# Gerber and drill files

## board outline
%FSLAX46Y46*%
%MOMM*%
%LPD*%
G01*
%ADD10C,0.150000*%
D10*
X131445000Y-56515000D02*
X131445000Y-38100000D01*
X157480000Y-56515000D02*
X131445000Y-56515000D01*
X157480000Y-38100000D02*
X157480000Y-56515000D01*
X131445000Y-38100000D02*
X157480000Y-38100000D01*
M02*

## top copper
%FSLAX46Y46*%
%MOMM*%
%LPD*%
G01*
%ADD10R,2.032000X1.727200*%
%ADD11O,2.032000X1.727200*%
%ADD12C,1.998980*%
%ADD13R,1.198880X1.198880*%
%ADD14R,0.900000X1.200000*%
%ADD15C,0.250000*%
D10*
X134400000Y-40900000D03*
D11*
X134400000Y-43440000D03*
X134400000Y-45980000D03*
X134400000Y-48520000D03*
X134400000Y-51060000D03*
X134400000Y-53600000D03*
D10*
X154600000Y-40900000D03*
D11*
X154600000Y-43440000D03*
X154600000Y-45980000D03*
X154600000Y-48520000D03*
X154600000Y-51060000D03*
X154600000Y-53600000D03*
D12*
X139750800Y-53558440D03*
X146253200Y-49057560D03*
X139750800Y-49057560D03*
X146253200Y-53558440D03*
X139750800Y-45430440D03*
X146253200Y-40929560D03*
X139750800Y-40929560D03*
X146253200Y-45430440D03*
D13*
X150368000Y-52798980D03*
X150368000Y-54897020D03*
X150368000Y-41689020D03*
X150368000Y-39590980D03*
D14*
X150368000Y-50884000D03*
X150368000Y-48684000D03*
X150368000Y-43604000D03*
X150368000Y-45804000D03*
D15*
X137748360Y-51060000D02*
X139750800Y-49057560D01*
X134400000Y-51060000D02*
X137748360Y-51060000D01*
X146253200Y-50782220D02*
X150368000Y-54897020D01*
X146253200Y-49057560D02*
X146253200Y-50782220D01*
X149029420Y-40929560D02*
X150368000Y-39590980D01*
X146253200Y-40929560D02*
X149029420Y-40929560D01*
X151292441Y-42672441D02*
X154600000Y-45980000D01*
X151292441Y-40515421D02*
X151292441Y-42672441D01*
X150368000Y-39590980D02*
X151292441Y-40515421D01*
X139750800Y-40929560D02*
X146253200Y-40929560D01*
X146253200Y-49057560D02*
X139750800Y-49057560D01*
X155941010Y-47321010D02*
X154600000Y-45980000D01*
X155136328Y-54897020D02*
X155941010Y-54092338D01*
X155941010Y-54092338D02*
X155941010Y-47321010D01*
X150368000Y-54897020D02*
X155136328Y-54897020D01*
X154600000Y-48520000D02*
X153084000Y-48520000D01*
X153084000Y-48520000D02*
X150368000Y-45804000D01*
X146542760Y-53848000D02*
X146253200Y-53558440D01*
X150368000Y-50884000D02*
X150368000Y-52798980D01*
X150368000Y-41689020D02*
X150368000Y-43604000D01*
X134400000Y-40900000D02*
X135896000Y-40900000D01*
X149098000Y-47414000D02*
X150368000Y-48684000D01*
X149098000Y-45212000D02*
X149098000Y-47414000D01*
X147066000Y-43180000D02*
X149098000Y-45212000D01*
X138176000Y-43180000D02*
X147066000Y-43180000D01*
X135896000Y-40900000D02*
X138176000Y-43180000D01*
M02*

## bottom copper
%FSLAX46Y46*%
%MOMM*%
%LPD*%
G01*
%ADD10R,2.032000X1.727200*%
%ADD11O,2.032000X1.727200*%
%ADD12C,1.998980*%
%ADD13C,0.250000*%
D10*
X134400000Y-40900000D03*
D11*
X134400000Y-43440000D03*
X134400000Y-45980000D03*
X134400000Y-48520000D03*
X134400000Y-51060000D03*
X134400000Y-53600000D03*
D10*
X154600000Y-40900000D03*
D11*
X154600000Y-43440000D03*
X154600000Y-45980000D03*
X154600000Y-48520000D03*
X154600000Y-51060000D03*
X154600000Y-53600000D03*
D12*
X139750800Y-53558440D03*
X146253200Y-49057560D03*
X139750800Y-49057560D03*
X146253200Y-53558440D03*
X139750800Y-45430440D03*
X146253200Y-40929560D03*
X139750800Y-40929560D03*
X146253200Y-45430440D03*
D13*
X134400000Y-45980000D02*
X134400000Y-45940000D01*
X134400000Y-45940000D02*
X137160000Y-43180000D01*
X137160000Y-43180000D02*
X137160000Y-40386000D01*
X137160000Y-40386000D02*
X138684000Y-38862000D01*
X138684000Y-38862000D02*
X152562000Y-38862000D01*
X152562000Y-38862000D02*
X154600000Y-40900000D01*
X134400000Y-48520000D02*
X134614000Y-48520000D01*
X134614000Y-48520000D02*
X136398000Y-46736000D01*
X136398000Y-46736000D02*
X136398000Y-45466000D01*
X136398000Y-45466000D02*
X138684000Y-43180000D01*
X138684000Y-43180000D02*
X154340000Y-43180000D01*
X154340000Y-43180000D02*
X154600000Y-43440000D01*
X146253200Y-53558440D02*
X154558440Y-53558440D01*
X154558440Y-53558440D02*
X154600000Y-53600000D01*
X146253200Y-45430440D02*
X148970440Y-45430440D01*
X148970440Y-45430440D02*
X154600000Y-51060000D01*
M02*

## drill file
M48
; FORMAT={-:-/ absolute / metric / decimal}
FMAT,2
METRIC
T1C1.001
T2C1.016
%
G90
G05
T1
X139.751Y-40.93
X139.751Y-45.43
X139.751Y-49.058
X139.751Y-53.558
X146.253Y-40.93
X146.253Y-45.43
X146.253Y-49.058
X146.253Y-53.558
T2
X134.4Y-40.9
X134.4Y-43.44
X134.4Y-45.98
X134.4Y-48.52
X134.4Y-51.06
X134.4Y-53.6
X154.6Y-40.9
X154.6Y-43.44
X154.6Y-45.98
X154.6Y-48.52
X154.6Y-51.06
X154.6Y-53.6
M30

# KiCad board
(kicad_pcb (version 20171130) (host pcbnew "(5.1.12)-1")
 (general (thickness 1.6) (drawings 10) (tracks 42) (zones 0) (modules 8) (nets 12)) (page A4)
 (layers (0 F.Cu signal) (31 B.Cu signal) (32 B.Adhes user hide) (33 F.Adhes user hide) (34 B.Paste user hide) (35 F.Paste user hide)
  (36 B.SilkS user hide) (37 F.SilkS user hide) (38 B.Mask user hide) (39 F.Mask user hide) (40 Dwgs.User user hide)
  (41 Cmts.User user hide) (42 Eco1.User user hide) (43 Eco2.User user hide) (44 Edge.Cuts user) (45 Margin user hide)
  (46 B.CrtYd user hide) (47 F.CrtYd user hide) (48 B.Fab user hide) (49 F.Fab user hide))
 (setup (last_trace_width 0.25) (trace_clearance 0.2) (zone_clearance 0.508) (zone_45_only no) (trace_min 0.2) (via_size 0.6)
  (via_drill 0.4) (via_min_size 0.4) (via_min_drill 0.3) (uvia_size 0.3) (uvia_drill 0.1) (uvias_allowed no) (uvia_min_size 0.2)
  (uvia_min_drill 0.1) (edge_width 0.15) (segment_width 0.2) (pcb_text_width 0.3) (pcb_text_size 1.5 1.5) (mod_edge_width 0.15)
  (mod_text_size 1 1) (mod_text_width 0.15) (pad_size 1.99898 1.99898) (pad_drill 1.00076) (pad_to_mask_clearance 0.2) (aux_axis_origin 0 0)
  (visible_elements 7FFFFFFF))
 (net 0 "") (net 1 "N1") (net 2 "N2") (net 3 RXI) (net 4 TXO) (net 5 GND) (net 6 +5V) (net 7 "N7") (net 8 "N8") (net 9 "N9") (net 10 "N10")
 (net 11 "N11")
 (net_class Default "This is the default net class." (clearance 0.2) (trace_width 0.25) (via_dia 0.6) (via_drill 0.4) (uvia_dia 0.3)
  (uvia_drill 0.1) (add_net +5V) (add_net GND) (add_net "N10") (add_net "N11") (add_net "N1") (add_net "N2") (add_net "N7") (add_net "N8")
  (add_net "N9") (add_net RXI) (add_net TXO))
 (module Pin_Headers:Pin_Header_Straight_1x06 (layer F.Cu) (at 134.4 40.9)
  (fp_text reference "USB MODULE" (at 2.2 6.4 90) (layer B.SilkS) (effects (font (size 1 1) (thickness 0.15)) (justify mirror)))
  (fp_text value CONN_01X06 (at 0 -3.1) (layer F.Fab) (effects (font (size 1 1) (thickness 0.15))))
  (pad 1 thru_hole rect (at 0 0) (size 2.032 1.7272) (drill 1.016) (layers *.Cu *.Mask F.SilkS) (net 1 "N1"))
  (pad 2 thru_hole oval (at 0 2.54) (size 2.032 1.7272) (drill 1.016) (layers *.Cu *.Mask F.SilkS) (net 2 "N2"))
  (pad 3 thru_hole oval (at 0 5.08) (size 2.032 1.7272) (drill 1.016) (layers *.Cu *.Mask F.SilkS) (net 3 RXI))
  (pad 4 thru_hole oval (at 0 7.62) (size 2.032 1.7272) (drill 1.016) (layers *.Cu *.Mask F.SilkS) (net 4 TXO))
  (pad 5 thru_hole oval (at 0 10.16) (size 2.032 1.7272) (drill 1.016) (layers *.Cu *.Mask F.SilkS) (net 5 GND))
  (pad 6 thru_hole oval (at 0 12.7) (size 2.032 1.7272) (drill 1.016) (layers *.Cu *.Mask F.SilkS) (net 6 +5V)))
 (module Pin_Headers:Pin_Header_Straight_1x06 (layer F.Cu) (at 154.6 40.9)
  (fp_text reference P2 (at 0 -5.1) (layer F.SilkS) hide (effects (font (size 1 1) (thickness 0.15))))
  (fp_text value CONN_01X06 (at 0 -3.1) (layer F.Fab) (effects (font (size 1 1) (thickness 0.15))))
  (pad 1 thru_hole rect (at 0 0) (size 2.032 1.7272) (drill 1.016) (layers *.Cu *.Mask F.SilkS) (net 3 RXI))
  (pad 2 thru_hole oval (at 0 2.54) (size 2.032 1.7272) (drill 1.016) (layers *.Cu *.Mask F.SilkS) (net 4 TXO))
  (pad 3 thru_hole oval (at 0 5.08) (size 2.032 1.7272) (drill 1.016) (layers *.Cu *.Mask F.SilkS) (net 5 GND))
  (pad 4 thru_hole oval (at 0 7.62) (size 2.032 1.7272) (drill 1.016) (layers *.Cu *.Mask F.SilkS) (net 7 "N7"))
  (pad 5 thru_hole oval (at 0 10.16) (size 2.032 1.7272) (drill 1.016) (layers *.Cu *.Mask F.SilkS) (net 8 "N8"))
  (pad 6 thru_hole oval (at 0 12.7) (size 2.032 1.7272) (drill 1.016) (layers *.Cu *.Mask F.SilkS) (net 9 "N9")))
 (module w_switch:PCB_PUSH (layer F.Cu) (at 143.002 51.308 90)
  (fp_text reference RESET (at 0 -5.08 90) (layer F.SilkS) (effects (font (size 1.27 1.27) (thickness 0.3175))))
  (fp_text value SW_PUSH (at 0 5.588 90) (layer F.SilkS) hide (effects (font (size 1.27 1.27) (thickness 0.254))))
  (pad 1 thru_hole circle (at -2.25044 -3.2512 90) (size 1.99898 1.99898) (drill 1.00076) (layers *.Cu *.Mask F.SilkS))
  (pad 2 thru_hole circle (at 2.25044 3.2512 90) (size 1.99898 1.99898) (drill 1.00076) (layers *.Cu *.Mask F.SilkS) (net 5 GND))
  (pad 4 thru_hole circle (at 2.25044 -3.2512 90) (size 1.99898 1.99898) (drill 1.00076) (layers *.Cu *.Mask F.SilkS) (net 5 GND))
  (pad 3 thru_hole circle (at -2.25044 3.2512 90) (size 1.99898 1.99898) (drill 1.00076) (layers *.Cu *.Mask F.SilkS) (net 9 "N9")))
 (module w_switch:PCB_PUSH (layer F.Cu) (at 143.002 43.18 90)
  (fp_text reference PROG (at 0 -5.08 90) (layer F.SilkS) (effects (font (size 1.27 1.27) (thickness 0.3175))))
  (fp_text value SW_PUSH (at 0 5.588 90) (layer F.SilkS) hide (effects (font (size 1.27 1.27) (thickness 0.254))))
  (pad 1 thru_hole circle (at -2.25044 -3.2512 90) (size 1.99898 1.99898) (drill 1.00076) (layers *.Cu *.Mask F.SilkS))
  (pad 2 thru_hole circle (at 2.25044 3.2512 90) (size 1.99898 1.99898) (drill 1.00076) (layers *.Cu *.Mask F.SilkS) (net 5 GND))
  (pad 4 thru_hole circle (at 2.25044 -3.2512 90) (size 1.99898 1.99898) (drill 1.00076) (layers *.Cu *.Mask F.SilkS) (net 5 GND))
  (pad 3 thru_hole circle (at -2.25044 3.2512 90) (size 1.99898 1.99898) (drill 1.00076) (layers *.Cu *.Mask F.SilkS) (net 8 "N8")))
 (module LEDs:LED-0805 (layer F.Cu) (at 150.368 53.848 90)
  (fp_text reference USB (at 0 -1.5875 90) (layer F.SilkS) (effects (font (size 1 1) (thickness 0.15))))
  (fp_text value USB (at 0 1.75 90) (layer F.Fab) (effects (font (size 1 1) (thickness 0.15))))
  (pad 2 smd rect (at 1.04902 0 270) (size 1.19888 1.19888) (layers F.Cu F.Paste F.Mask) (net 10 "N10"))
  (pad 1 smd rect (at -1.04902 0 270) (size 1.19888 1.19888) (layers F.Cu F.Paste F.Mask) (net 5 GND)))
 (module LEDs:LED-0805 (layer F.Cu) (at 150.368 40.64 270)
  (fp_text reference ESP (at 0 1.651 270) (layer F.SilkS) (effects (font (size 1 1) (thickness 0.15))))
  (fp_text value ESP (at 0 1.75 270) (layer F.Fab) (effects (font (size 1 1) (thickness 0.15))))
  (pad 2 smd rect (at 1.04902 0 90) (size 1.19888 1.19888) (layers F.Cu F.Paste F.Mask) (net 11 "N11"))
  (pad 1 smd rect (at -1.04902 0 90) (size 1.19888 1.19888) (layers F.Cu F.Paste F.Mask) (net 5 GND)))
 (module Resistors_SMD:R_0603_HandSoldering (layer F.Cu) (at 150.368 49.784 90)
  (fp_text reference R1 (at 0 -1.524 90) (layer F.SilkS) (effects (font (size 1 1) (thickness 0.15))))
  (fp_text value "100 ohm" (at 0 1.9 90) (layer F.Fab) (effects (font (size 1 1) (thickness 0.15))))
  (pad 1 smd rect (at -1.1 0 90) (size 1.2 0.9) (layers F.Cu F.Paste F.Mask) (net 10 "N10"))
  (pad 2 smd rect (at 1.1 0 90) (size 1.2 0.9) (layers F.Cu F.Paste F.Mask) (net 1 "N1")))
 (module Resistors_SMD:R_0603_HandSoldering (layer F.Cu) (at 150.368 44.704 270)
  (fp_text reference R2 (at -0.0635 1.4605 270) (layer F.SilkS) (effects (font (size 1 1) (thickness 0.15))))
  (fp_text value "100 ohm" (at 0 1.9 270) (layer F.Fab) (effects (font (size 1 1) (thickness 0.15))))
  (pad 1 smd rect (at -1.1 0 270) (size 1.2 0.9) (layers F.Cu F.Paste F.Mask) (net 11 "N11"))
  (pad 2 smd rect (at 1.1 0 270) (size 1.2 0.9) (layers F.Cu F.Paste F.Mask) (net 7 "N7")))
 (gr_line (start 131.445 56.515) (end 131.445 38.1) (angle 90) (layer Edge.Cuts) (width 0.15))
 (gr_line (start 157.48 56.515) (end 131.445 56.515) (angle 90) (layer Edge.Cuts) (width 0.15))
 (gr_line (start 157.48 38.1) (end 157.48 56.515) (angle 90) (layer Edge.Cuts) (width 0.15))
 (gr_line (start 131.445 38.1) (end 157.48 38.1) (angle 90) (layer Edge.Cuts) (width 0.15))
 (segment (start 134.4 45.98) (end 134.4 45.94) (width 0.25) (layer B.Cu) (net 3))
 (segment (start 134.4 45.94) (end 137.16 43.18) (width 0.25) (layer B.Cu) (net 3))
 (segment (start 137.16 43.18) (end 137.16 40.386) (width 0.25) (layer B.Cu) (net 3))
 (segment (start 137.16 40.386) (end 138.684 38.862) (width 0.25) (layer B.Cu) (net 3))
 (segment (start 138.684 38.862) (end 152.562 38.862) (width 0.25) (layer B.Cu) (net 3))
 (segment (start 152.562 38.862) (end 154.6 40.9) (width 0.25) (layer B.Cu) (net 3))
 (segment (start 134.4 48.52) (end 134.614 48.52) (width 0.25) (layer B.Cu) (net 4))
 (segment (start 134.614 48.52) (end 136.398 46.736) (width 0.25) (layer B.Cu) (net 4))
 (segment (start 136.398 46.736) (end 136.398 45.466) (width 0.25) (layer B.Cu) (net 4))
 (segment (start 136.398 45.466) (end 138.684 43.18) (width 0.25) (layer B.Cu) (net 4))
 (segment (start 138.684 43.18) (end 154.34 43.18) (width 0.25) (layer B.Cu) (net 4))
 (segment (start 154.34 43.18) (end 154.6 43.44) (width 0.25) (layer B.Cu) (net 4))
 (segment (start 137.74836 51.06) (end 139.7508 49.05756) (width 0.25) (layer F.Cu) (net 5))
 (segment (start 134.4 51.06) (end 137.74836 51.06) (width 0.25) (layer F.Cu) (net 5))
 (segment (start 146.2532 50.78222) (end 150.368 54.89702) (width 0.25) (layer F.Cu) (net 5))
 (segment (start 146.2532 49.05756) (end 146.2532 50.78222) (width 0.25) (layer F.Cu) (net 5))
 (segment (start 149.02942 40.92956) (end 150.368 39.59098) (width 0.25) (layer F.Cu) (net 5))
 (segment (start 146.2532 40.92956) (end 149.02942 40.92956) (width 0.25) (layer F.Cu) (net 5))
 (segment (start 151.292441 42.672441) (end 154.6 45.98) (width 0.25) (layer F.Cu) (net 5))
 (segment (start 151.292441 40.515421) (end 151.292441 42.672441) (width 0.25) (layer F.Cu) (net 5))
 (segment (start 150.368 39.59098) (end 151.292441 40.515421) (width 0.25) (layer F.Cu) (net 5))
 (segment (start 139.7508 40.92956) (end 146.2532 40.92956) (width 0.25) (layer F.Cu) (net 5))
 (segment (start 146.2532 49.05756) (end 139.7508 49.05756) (width 0.25) (layer F.Cu) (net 5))
 (segment (start 155.94101 47.32101) (end 154.6 45.98) (width 0.25) (layer F.Cu) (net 5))
 (segment (start 155.136328 54.89702) (end 155.94101 54.092338) (width 0.25) (layer F.Cu) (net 5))
 (segment (start 155.94101 54.092338) (end 155.94101 47.32101) (width 0.25) (layer F.Cu) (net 5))
 (segment (start 150.368 54.89702) (end 155.136328 54.89702) (width 0.25) (layer F.Cu) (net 5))
 (segment (start 154.6 48.52) (end 153.084 48.52) (width 0.25) (layer F.Cu) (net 7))
 (segment (start 153.084 48.52) (end 150.368 45.804) (width 0.25) (layer F.Cu) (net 7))
 (segment (start 146.2532 53.55844) (end 154.55844 53.55844) (width 0.25) (layer B.Cu) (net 9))
 (segment (start 154.55844 53.55844) (end 154.6 53.6) (width 0.25) (layer B.Cu) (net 9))
 (segment (start 146.54276 53.848) (end 146.2532 53.55844) (width 0.25) (layer F.Cu) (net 9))
 (segment (start 146.2532 45.43044) (end 148.97044 45.43044) (width 0.25) (layer B.Cu) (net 8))
 (segment (start 148.97044 45.43044) (end 154.6 51.06) (width 0.25) (layer B.Cu) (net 8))
 (segment (start 150.368 50.884) (end 150.368 52.79898) (width 0.25) (layer F.Cu) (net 10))
 (segment (start 150.368 41.68902) (end 150.368 43.604) (width 0.25) (layer F.Cu) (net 11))
 (segment (start 134.4 40.9) (end 135.896 40.9) (width 0.25) (layer F.Cu) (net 1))
 (segment (start 149.098 47.414) (end 150.368 48.684) (width 0.25) (layer F.Cu) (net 1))
 (segment (start 149.098 45.212) (end 149.098 47.414) (width 0.25) (layer F.Cu) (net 1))
 (segment (start 147.066 43.18) (end 149.098 45.212) (width 0.25) (layer F.Cu) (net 1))
 (segment (start 138.176 43.18) (end 147.066 43.18) (width 0.25) (layer F.Cu) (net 1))
 (segment (start 135.896 40.9) (end 138.176 43.18) (width 0.25) (layer F.Cu) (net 1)))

